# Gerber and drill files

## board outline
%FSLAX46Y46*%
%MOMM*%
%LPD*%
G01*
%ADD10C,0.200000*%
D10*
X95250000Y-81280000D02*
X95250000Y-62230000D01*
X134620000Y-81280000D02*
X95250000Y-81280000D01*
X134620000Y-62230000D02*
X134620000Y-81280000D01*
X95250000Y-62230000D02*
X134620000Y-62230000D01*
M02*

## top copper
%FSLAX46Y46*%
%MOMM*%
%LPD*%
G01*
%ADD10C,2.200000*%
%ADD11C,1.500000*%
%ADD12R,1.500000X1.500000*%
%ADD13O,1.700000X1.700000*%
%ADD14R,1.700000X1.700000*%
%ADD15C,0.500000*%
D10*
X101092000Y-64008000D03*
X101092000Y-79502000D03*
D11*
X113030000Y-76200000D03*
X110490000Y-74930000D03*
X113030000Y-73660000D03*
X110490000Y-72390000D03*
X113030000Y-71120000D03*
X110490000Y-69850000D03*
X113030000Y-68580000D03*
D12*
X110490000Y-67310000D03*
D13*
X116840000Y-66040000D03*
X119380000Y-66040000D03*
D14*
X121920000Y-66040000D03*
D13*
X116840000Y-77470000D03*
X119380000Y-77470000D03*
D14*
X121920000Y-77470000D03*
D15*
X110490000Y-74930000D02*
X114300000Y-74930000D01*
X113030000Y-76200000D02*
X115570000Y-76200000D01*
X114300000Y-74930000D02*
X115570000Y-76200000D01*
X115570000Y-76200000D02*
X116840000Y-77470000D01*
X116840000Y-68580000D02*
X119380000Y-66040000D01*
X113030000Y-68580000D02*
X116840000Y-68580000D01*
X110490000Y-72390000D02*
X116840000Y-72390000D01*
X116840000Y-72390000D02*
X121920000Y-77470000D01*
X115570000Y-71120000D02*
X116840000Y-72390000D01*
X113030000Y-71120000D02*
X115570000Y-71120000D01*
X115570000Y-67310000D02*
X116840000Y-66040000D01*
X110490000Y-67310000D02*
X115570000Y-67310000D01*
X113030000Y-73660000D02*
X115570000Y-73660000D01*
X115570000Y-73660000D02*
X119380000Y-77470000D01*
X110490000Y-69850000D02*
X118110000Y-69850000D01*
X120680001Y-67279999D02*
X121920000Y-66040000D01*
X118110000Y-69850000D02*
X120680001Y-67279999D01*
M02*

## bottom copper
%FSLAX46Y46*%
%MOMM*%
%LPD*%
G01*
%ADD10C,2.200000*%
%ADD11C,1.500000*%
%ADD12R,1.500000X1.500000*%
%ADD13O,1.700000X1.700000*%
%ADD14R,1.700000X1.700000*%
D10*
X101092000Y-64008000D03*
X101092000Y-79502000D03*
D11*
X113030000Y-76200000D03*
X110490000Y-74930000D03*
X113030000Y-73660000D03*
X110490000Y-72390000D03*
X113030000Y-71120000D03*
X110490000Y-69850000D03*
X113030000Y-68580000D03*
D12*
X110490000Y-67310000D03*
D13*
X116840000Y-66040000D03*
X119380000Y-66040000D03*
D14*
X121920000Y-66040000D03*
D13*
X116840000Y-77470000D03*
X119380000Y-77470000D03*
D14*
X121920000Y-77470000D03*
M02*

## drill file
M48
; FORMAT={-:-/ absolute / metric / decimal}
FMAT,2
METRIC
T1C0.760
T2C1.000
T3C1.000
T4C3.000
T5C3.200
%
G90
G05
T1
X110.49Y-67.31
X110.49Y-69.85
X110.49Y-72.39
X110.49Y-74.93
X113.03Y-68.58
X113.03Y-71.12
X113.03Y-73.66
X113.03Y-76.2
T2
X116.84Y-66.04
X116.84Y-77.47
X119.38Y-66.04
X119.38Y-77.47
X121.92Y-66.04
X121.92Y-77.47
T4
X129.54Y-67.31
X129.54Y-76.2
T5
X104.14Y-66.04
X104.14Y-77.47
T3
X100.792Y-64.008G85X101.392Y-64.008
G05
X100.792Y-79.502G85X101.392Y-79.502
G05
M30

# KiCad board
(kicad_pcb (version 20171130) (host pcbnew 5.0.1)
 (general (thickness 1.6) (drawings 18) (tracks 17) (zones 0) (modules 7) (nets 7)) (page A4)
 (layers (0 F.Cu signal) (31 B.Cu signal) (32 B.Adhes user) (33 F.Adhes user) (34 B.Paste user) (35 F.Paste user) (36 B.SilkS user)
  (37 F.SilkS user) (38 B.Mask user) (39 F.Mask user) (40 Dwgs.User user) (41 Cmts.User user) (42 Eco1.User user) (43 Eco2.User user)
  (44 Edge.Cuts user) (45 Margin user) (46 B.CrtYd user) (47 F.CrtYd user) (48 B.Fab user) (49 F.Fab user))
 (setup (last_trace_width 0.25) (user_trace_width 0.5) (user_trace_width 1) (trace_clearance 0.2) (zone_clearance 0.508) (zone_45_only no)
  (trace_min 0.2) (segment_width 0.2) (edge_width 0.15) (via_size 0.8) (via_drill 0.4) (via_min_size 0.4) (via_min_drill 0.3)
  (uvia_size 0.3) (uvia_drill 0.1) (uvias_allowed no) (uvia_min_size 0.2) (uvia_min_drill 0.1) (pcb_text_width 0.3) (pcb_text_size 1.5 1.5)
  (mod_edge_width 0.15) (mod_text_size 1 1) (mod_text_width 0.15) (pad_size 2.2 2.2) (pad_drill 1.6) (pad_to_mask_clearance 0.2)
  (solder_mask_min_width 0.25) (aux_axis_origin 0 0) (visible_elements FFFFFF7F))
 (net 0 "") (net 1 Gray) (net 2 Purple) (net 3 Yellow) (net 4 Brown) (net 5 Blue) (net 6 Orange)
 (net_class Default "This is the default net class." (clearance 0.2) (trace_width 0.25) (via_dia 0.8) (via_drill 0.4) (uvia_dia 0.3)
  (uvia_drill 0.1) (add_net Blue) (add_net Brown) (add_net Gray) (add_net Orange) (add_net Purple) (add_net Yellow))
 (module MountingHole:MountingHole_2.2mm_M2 (layer F.Cu) (at 101.092 64.008)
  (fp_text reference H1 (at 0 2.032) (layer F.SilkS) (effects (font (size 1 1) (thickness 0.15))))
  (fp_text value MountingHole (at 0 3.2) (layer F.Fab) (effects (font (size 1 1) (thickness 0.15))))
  (pad "" np_thru_hole circle (at 0 0) (size 2.2 2.2) (drill oval 1.6 1) (layers *.Cu *.Mask)))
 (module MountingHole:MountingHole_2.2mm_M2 (layer F.Cu) (at 101.092 79.502)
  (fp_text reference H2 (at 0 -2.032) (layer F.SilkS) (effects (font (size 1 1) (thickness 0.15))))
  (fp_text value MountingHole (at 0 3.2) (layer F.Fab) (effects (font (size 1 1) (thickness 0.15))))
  (pad "" np_thru_hole circle (at 0 0) (size 2.2 2.2) (drill oval 1.6 1) (layers *.Cu *.Mask)))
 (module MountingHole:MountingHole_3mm (layer F.Cu) (at 129.54 67.31)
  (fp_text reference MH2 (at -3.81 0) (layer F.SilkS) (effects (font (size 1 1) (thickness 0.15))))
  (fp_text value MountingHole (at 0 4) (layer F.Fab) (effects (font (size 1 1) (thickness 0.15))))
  (pad 1 np_thru_hole circle (at 0 0) (size 3 3) (drill 3) (layers *.Cu *.Mask)))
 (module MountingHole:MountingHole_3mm (layer F.Cu) (at 129.54 76.2)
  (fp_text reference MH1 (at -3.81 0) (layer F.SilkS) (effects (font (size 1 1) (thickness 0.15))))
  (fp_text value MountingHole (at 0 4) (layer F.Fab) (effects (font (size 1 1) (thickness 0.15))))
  (pad 1 np_thru_hole circle (at 0 0) (size 3 3) (drill 3) (layers *.Cu *.Mask)))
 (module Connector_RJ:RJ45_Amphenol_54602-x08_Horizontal (layer F.Cu) (at 110.49 67.31 270)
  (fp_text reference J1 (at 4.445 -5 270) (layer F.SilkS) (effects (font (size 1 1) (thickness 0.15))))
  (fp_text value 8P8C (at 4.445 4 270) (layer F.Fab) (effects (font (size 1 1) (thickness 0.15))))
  (pad 8 thru_hole circle (at 8.89 -2.54 270) (size 1.5 1.5) (drill 0.76) (layers *.Cu *.Mask) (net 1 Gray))
  (pad 7 thru_hole circle (at 7.62 0 270) (size 1.5 1.5) (drill 0.76) (layers *.Cu *.Mask) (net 1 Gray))
  (pad 6 thru_hole circle (at 6.35 -2.54 270) (size 1.5 1.5) (drill 0.76) (layers *.Cu *.Mask) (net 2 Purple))
  (pad 5 thru_hole circle (at 5.08 0 270) (size 1.5 1.5) (drill 0.76) (layers *.Cu *.Mask) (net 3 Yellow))
  (pad 4 thru_hole circle (at 3.81 -2.54 270) (size 1.5 1.5) (drill 0.76) (layers *.Cu *.Mask) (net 3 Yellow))
  (pad 3 thru_hole circle (at 2.54 0 270) (size 1.5 1.5) (drill 0.76) (layers *.Cu *.Mask) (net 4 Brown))
  (pad 2 thru_hole circle (at 1.27 -2.54 270) (size 1.5 1.5) (drill 0.76) (layers *.Cu *.Mask) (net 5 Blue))
  (pad 1 thru_hole rect (at 0 0 270) (size 1.5 1.5) (drill 0.76) (layers *.Cu *.Mask) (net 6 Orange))
  (pad "" np_thru_hole circle (at -1.27 6.35 270) (size 3.2 3.2) (drill 3.2) (layers *.Cu *.Mask))
  (pad "" np_thru_hole circle (at 10.16 6.35 270) (size 3.2 3.2) (drill 3.2) (layers *.Cu *.Mask)))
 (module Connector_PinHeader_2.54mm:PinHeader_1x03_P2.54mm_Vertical (layer F.Cu) (at 121.92 66.04 270)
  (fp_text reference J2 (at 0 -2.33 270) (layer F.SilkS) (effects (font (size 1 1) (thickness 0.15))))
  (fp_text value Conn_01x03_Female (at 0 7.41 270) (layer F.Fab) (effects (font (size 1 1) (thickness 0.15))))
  (pad 3 thru_hole oval (at 0 5.08 270) (size 1.7 1.7) (drill 1) (layers *.Cu *.Mask) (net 6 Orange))
  (pad 2 thru_hole oval (at 0 2.54 270) (size 1.7 1.7) (drill 1) (layers *.Cu *.Mask) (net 5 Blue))
  (pad 1 thru_hole rect (at 0 0 270) (size 1.7 1.7) (drill 1) (layers *.Cu *.Mask) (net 4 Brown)))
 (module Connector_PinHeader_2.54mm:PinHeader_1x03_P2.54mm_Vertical (layer F.Cu) (at 121.92 77.47 270)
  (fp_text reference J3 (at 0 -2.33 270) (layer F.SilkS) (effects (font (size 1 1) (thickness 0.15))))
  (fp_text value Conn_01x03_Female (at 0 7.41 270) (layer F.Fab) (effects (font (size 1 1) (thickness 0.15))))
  (pad 3 thru_hole oval (at 0 5.08 270) (size 1.7 1.7) (drill 1) (layers *.Cu *.Mask) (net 1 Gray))
  (pad 2 thru_hole oval (at 0 2.54 270) (size 1.7 1.7) (drill 1) (layers *.Cu *.Mask) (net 2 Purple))
  (pad 1 thru_hole rect (at 0 0 270) (size 1.7 1.7) (drill 1) (layers *.Cu *.Mask) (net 3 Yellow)))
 (gr_line (start 95.25 81.28) (end 95.25 62.23) (layer Edge.Cuts) (width 0.2))
 (gr_line (start 134.62 81.28) (end 95.25 81.28) (layer Edge.Cuts) (width 0.2))
 (gr_line (start 134.62 62.23) (end 134.62 81.28) (layer Edge.Cuts) (width 0.2))
 (gr_line (start 95.25 62.23) (end 134.62 62.23) (layer Edge.Cuts) (width 0.2))
 (segment (start 110.49 74.93) (end 114.3 74.93) (width 0.5) (layer F.Cu) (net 1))
 (segment (start 113.03 76.2) (end 115.57 76.2) (width 0.5) (layer F.Cu) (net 1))
 (segment (start 114.3 74.93) (end 115.57 76.2) (width 0.5) (layer F.Cu) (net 1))
 (segment (start 115.57 76.2) (end 116.84 77.47) (width 0.5) (layer F.Cu) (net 1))
 (segment (start 116.84 68.58) (end 119.38 66.04) (width 0.5) (layer F.Cu) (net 5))
 (segment (start 113.03 68.58) (end 116.84 68.58) (width 0.5) (layer F.Cu) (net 5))
 (segment (start 110.49 72.39) (end 116.84 72.39) (width 0.5) (layer F.Cu) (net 3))
 (segment (start 116.84 72.39) (end 121.92 77.47) (width 0.5) (layer F.Cu) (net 3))
 (segment (start 115.57 71.12) (end 116.84 72.39) (width 0.5) (layer F.Cu) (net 3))
 (segment (start 113.03 71.12) (end 115.57 71.12) (width 0.5) (layer F.Cu) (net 3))
 (segment (start 115.57 67.31) (end 116.84 66.04) (width 0.5) (layer F.Cu) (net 6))
 (segment (start 110.49 67.31) (end 115.57 67.31) (width 0.5) (layer F.Cu) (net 6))
 (segment (start 113.03 73.66) (end 115.57 73.66) (width 0.5) (layer F.Cu) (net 2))
 (segment (start 115.57 73.66) (end 119.38 77.47) (width 0.5) (layer F.Cu) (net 2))
 (segment (start 110.49 69.85) (end 118.11 69.85) (width 0.5) (layer F.Cu) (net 4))
 (segment (start 120.680001 67.279999) (end 121.92 66.04) (width 0.5) (layer F.Cu) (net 4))
 (segment (start 118.11 69.85) (end 120.680001 67.279999) (width 0.5) (layer F.Cu) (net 4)))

